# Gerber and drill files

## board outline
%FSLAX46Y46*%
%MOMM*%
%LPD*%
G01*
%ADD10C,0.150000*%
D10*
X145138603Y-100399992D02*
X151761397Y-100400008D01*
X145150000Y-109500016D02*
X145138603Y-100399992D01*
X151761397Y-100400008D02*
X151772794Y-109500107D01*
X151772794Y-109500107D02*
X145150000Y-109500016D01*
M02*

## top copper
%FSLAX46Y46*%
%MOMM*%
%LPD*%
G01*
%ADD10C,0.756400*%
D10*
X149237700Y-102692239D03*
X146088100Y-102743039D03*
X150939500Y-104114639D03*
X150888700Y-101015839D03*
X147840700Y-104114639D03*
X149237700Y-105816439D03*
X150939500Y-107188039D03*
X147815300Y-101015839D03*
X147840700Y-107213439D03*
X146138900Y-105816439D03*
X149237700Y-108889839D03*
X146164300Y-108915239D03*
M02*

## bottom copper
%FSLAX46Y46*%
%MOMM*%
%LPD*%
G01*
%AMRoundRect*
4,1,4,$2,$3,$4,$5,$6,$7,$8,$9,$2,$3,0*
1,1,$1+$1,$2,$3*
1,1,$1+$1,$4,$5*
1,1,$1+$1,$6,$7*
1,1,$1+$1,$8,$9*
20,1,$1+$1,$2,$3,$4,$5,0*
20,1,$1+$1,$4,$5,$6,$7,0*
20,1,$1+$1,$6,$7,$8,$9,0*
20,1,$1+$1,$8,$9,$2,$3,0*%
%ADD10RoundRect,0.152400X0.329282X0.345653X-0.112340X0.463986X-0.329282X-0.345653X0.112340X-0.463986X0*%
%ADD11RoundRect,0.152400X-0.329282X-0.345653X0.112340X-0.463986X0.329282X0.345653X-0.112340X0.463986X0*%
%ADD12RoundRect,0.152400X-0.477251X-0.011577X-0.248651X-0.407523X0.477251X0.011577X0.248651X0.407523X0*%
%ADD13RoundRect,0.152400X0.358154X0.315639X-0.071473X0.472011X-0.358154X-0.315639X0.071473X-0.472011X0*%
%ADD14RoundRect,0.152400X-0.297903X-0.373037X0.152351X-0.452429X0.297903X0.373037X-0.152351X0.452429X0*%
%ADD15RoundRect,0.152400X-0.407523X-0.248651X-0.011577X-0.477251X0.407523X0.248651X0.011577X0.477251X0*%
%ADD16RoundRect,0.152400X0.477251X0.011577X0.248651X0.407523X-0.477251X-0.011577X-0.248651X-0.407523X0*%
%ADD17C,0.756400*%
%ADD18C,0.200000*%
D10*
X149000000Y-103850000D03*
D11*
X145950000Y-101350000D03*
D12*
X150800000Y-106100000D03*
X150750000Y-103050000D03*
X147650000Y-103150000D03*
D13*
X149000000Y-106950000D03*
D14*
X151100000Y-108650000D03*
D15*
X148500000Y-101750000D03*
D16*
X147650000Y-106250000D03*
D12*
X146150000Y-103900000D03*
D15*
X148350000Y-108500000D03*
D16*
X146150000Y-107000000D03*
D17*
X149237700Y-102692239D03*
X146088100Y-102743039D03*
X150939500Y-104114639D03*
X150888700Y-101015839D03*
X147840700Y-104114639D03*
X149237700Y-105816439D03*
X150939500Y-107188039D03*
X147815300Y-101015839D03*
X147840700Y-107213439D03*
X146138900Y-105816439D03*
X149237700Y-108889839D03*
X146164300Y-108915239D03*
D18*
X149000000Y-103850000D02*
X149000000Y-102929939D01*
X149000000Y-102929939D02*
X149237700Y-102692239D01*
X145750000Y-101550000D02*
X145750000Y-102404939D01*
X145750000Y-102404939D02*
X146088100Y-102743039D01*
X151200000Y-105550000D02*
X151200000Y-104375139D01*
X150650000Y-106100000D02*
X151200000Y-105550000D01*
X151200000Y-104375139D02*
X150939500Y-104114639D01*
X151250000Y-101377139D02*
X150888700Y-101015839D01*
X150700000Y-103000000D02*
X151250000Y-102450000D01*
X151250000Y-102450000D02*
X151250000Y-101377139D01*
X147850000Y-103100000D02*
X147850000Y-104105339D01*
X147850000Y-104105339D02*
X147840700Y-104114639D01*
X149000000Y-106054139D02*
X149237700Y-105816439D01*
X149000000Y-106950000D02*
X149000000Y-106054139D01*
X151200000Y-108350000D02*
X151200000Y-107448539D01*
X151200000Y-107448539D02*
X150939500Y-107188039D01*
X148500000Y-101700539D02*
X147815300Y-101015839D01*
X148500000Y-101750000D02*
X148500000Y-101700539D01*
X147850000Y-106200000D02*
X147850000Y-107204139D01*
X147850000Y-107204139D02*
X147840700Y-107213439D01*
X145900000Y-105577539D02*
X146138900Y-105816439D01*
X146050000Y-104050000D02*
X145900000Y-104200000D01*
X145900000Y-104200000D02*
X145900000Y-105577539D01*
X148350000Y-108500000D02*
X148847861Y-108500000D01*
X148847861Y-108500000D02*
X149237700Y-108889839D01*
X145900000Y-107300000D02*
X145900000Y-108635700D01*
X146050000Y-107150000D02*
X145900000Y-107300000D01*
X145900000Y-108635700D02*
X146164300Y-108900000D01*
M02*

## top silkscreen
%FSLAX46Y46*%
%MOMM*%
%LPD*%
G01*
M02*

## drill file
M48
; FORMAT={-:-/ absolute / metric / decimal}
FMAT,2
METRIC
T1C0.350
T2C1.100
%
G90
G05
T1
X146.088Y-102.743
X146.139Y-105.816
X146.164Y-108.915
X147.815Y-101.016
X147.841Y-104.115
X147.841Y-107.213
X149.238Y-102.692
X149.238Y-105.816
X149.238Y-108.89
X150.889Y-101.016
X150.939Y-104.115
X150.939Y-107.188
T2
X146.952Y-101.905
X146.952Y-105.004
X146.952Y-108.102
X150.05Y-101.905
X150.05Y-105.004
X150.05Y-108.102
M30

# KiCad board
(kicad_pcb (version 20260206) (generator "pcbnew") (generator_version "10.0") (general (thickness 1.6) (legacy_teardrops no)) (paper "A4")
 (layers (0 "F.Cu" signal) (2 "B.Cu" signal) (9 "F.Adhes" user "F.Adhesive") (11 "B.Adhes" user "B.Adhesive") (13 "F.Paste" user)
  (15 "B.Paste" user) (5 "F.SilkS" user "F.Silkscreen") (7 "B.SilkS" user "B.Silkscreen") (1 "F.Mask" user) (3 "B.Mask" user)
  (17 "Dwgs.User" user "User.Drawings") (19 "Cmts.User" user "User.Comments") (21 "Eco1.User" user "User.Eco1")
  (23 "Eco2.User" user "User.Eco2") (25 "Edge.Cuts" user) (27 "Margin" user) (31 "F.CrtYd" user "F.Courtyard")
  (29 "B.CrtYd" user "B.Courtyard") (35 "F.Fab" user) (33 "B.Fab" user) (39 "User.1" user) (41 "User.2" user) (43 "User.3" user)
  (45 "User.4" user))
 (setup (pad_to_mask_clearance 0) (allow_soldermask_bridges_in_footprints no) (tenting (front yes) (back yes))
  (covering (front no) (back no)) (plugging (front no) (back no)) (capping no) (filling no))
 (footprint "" (layer "F.Cu") (at 149 103.85 180)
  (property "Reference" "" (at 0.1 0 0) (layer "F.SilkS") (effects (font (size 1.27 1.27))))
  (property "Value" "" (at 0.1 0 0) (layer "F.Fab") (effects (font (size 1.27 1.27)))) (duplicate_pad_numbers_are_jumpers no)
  (pad "4B" smd roundrect (at 0 0 165) (size 0.762 1.143) (layers "B.Cu" "B.Mask" "B.Paste") (roundrect_rratio 0.2) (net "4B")))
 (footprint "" (layer "F.Cu") (at 145.95 101.35)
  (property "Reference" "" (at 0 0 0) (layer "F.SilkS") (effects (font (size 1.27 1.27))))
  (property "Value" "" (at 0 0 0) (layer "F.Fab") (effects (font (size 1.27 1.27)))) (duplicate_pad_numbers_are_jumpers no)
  (pad "1B" smd roundrect (at 0 0 345) (size 0.762 1.143) (layers "B.Cu" "B.Mask" "B.Paste") (roundrect_rratio 0.2) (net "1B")))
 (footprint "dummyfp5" (layer "F.Cu") (at 150.0505 108.102439)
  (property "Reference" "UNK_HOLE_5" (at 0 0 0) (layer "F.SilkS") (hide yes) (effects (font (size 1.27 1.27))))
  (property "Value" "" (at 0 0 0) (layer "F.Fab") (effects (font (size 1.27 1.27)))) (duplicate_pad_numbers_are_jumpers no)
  (pad "" np_thru_hole circle (at 0 0) (size 1.1 1.1) (drill 1.1) (layers "*.Cu" "*.Mask")))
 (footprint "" (layer "F.Cu") (at 150.8 106.1)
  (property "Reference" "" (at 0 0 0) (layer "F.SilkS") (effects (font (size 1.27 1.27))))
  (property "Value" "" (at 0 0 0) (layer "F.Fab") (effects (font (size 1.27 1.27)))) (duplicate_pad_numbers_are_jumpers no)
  (pad "5A" smd roundrect (at 0 0 300) (size 0.762 1.143) (layers "B.Cu" "B.Mask" "B.Paste") (roundrect_rratio 0.2) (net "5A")))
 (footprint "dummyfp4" (layer "F.Cu") (at 146.9517 108.102439)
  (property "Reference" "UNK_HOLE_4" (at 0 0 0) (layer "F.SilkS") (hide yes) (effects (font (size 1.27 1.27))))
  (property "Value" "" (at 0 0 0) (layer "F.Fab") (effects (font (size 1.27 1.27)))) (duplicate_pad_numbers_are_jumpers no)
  (pad "" np_thru_hole circle (at 0 0) (size 1.1 1.1) (drill 1.1) (layers "*.Cu" "*.Mask")))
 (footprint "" (layer "F.Cu") (at 150.75 103.05)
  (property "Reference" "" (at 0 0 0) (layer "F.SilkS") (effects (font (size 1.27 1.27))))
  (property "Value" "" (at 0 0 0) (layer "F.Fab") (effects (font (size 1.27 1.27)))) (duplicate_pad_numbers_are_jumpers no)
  (pad "4A" smd roundrect (at 0 0 300) (size 0.762 1.143) (layers "B.Cu" "B.Mask" "B.Paste") (roundrect_rratio 0.2) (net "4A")))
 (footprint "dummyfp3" (layer "F.Cu") (at 150.0505 105.003639)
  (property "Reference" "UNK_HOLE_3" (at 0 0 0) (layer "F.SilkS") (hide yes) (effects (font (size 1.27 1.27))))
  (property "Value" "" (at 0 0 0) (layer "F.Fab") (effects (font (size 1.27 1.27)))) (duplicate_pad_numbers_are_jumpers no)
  (pad "" np_thru_hole circle (at 0 0) (size 1.1 1.1) (drill 1.1) (layers "*.Cu" "*.Mask")))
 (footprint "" (layer "F.Cu") (at 147.65 103.15 -90)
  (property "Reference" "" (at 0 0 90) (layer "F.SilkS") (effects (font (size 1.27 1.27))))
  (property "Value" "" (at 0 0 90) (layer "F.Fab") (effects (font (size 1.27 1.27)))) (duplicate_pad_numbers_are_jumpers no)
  (pad "2A" smd roundrect (at 0 0 300) (size 0.762 1.143) (layers "B.Cu" "B.Mask" "B.Paste") (roundrect_rratio 0.2) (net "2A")))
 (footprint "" (layer "F.Cu") (at 149 106.95 180)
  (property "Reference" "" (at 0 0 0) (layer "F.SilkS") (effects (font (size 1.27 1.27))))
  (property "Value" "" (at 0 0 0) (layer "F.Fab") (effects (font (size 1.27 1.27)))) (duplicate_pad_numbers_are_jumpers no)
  (pad "5B" smd roundrect (at 0 0 160) (size 0.762 1.143) (layers "B.Cu" "B.Mask" "B.Paste") (roundrect_rratio 0.2) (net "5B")))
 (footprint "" (layer "F.Cu") (at 151.1 108.65)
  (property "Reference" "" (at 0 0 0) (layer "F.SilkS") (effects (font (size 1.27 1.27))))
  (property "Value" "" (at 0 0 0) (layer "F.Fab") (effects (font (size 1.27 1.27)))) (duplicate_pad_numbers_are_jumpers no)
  (pad "6A" smd roundrect (at 0 0 350) (size 0.762 1.143) (layers "B.Cu" "B.Mask" "B.Paste") (roundrect_rratio 0.2) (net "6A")))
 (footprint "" (layer "F.Cu") (at 148.5 101.75)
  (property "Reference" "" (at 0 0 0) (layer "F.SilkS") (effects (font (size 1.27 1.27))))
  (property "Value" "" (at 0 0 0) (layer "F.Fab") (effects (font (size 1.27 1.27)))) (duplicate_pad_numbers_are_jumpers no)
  (pad "1A" smd roundrect (at 0 0 330) (size 0.762 1.143) (layers "B.Cu" "B.Mask" "B.Paste") (roundrect_rratio 0.2) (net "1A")))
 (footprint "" (layer "F.Cu") (at 147.65 106.25 90)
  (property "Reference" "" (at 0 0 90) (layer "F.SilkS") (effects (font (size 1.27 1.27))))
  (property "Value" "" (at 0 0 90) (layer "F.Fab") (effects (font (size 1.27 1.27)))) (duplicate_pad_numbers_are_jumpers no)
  (pad "3A" smd roundrect (at 0 0 120) (size 0.762 1.143) (layers "B.Cu" "B.Mask" "B.Paste") (roundrect_rratio 0.2) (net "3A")))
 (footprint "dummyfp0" (layer "F.Cu") (at 146.9517 101.904839)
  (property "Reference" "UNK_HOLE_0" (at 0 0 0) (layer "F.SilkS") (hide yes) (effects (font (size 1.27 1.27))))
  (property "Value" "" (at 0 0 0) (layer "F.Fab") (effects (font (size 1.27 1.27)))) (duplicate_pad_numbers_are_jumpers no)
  (pad "" np_thru_hole circle (at 0 0) (size 1.1 1.1) (drill 1.1) (layers "*.Cu" "*.Mask")))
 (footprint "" (layer "F.Cu") (at 146.15 103.9)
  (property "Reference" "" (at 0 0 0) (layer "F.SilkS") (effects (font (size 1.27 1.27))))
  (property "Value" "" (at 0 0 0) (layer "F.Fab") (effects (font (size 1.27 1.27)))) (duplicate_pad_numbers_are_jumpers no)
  (pad "2B" smd roundrect (at 0 0 300) (size 0.762 1.143) (layers "B.Cu" "B.Mask" "B.Paste") (roundrect_rratio 0.2) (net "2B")))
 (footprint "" (layer "F.Cu") (at 148.35 108.5)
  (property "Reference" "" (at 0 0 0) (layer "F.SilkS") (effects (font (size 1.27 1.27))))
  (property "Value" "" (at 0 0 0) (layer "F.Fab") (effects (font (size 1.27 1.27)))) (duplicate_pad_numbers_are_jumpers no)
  (pad "6B" smd roundrect (at 0 0 330) (size 0.762 1.143) (layers "B.Cu" "B.Mask" "B.Paste") (roundrect_rratio 0.2) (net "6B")))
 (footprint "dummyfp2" (layer "F.Cu") (at 146.9517 105.003639)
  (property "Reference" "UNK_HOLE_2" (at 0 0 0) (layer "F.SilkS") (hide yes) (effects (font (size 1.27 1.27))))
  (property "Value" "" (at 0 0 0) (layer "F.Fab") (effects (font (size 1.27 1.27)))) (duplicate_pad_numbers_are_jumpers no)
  (pad "" np_thru_hole circle (at 0 0) (size 1.1 1.1) (drill 1.1) (layers "*.Cu" "*.Mask")))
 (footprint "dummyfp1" (layer "F.Cu") (at 150.0505 101.904839)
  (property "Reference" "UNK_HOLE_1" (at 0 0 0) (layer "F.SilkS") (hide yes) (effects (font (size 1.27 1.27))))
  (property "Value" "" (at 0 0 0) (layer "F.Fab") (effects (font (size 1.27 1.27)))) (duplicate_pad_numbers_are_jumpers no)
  (pad "" np_thru_hole circle (at 0 0) (size 1.1 1.1) (drill 1.1) (layers "*.Cu" "*.Mask")))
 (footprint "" (layer "F.Cu") (at 146.15 107 180)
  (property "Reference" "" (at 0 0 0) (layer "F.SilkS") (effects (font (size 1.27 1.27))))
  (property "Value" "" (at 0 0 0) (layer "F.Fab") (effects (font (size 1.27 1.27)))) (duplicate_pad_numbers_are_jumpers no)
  (pad "3B" smd roundrect (at 0 0 120) (size 0.762 1.143) (layers "B.Cu" "B.Mask" "B.Paste") (roundrect_rratio 0.2) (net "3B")))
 (gr_line (start 145.138603 100.399992) (end 151.761397 100.400008) (stroke (width 0.15) (type solid)) (layer "Edge.Cuts"))
 (gr_line (start 145.15 109.500016) (end 145.138603 100.399992) (stroke (width 0.15) (type solid)) (layer "Edge.Cuts"))
 (gr_line (start 151.761397 100.400008) (end 151.772794 109.500107) (stroke (width 0.15) (type solid)) (layer "Edge.Cuts"))
 (gr_line (start 151.772794 109.500107) (end 145.15 109.500016) (stroke (width 0.15) (type solid)) (layer "Edge.Cuts"))
 (via (at 149.2377 102.692239) (size 0.7564) (drill 0.35) (layers "F.Cu" "B.Cu") (free yes) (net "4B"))
 (segment (start 149 103.85) (end 149 102.929939) (width 0.2) (layer "B.Cu") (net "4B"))
 (segment (start 149 102.929939) (end 149.2377 102.692239) (width 0.2) (layer "B.Cu") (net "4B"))
 (via (at 146.0881 102.743039) (size 0.7564) (drill 0.35) (layers "F.Cu" "B.Cu") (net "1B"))
 (segment (start 145.75 101.55) (end 145.75 102.404939) (width 0.2) (layer "B.Cu") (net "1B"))
 (segment (start 145.75 102.404939) (end 146.0881 102.743039) (width 0.2) (layer "B.Cu") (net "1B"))
 (via (at 150.9395 104.114639) (size 0.7564) (drill 0.35) (layers "F.Cu" "B.Cu") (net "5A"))
 (segment (start 151.2 105.55) (end 151.2 104.375139) (width 0.2) (layer "B.Cu") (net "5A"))
 (segment (start 150.65 106.1) (end 151.2 105.55) (width 0.2) (layer "B.Cu") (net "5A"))
 (segment (start 151.2 104.375139) (end 150.9395 104.114639) (width 0.2) (layer "B.Cu") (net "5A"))
 (via (at 150.8887 101.015839) (size 0.7564) (drill 0.35) (layers "F.Cu" "B.Cu") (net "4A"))
 (segment (start 151.25 101.377139) (end 150.8887 101.015839) (width 0.2) (layer "B.Cu") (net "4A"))
 (segment (start 150.7 103) (end 151.25 102.45) (width 0.2) (layer "B.Cu") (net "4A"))
 (segment (start 151.25 102.45) (end 151.25 101.377139) (width 0.2) (layer "B.Cu") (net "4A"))
 (via (at 147.8407 104.114639) (size 0.7564) (drill 0.35) (layers "F.Cu" "B.Cu") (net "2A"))
 (segment (start 147.85 103.1) (end 147.85 104.105339) (width 0.2) (layer "B.Cu") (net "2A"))
 (segment (start 147.85 104.105339) (end 147.8407 104.114639) (width 0.2) (layer "B.Cu") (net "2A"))
 (via (at 149.2377 105.816439) (size 0.7564) (drill 0.35) (layers "F.Cu" "B.Cu") (free yes) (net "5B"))
 (segment (start 149 106.054139) (end 149.2377 105.816439) (width 0.2) (layer "B.Cu") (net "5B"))
 (segment (start 149 106.95) (end 149 106.054139) (width 0.2) (layer "B.Cu") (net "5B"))
 (via (at 150.9395 107.188039) (size 0.7564) (drill 0.35) (layers "F.Cu" "B.Cu") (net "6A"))
 (segment (start 151.2 108.35) (end 151.2 107.448539) (width 0.2) (layer "B.Cu") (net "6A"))
 (segment (start 151.2 107.448539) (end 150.9395 107.188039) (width 0.2) (layer "B.Cu") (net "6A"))
 (via (at 147.8153 101.015839) (size 0.7564) (drill 0.35) (layers "F.Cu" "B.Cu") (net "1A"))
 (segment (start 148.5 101.700539) (end 147.8153 101.015839) (width 0.2) (layer "B.Cu") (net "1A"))
 (segment (start 148.5 101.75) (end 148.5 101.700539) (width 0.2) (layer "B.Cu") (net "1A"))
 (via (at 147.8407 107.213439) (size 0.7564) (drill 0.35) (layers "F.Cu" "B.Cu") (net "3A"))
 (segment (start 147.85 106.2) (end 147.85 107.204139) (width 0.2) (layer "B.Cu") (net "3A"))
 (segment (start 147.85 107.204139) (end 147.8407 107.213439) (width 0.2) (layer "B.Cu") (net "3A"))
 (via (at 146.1389 105.816439) (size 0.7564) (drill 0.35) (layers "F.Cu" "B.Cu") (free yes) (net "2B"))
 (segment (start 145.9 105.577539) (end 146.1389 105.816439) (width 0.2) (layer "B.Cu") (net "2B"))
 (segment (start 146.05 104.05) (end 145.9 104.2) (width 0.2) (layer "B.Cu") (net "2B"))
 (segment (start 145.9 104.2) (end 145.9 105.577539) (width 0.2) (layer "B.Cu") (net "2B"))
 (via (at 149.2377 108.889839) (size 0.7564) (drill 0.35) (layers "F.Cu" "B.Cu") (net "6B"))
 (segment (start 148.35 108.5) (end 148.847861 108.5) (width 0.2) (layer "B.Cu") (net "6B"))
 (segment (start 148.847861 108.5) (end 149.2377 108.889839) (width 0.2) (layer "B.Cu") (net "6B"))
 (via (at 146.1643 108.915239) (size 0.7564) (drill 0.35) (layers "F.Cu" "B.Cu") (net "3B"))
 (segment (start 145.9 107.3) (end 145.9 108.6357) (width 0.2) (layer "B.Cu") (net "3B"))
 (segment (start 146.05 107.15) (end 145.9 107.3) (width 0.2) (layer "B.Cu") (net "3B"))
 (segment (start 145.9 108.6357) (end 146.1643 108.9) (width 0.2) (layer "B.Cu") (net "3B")))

